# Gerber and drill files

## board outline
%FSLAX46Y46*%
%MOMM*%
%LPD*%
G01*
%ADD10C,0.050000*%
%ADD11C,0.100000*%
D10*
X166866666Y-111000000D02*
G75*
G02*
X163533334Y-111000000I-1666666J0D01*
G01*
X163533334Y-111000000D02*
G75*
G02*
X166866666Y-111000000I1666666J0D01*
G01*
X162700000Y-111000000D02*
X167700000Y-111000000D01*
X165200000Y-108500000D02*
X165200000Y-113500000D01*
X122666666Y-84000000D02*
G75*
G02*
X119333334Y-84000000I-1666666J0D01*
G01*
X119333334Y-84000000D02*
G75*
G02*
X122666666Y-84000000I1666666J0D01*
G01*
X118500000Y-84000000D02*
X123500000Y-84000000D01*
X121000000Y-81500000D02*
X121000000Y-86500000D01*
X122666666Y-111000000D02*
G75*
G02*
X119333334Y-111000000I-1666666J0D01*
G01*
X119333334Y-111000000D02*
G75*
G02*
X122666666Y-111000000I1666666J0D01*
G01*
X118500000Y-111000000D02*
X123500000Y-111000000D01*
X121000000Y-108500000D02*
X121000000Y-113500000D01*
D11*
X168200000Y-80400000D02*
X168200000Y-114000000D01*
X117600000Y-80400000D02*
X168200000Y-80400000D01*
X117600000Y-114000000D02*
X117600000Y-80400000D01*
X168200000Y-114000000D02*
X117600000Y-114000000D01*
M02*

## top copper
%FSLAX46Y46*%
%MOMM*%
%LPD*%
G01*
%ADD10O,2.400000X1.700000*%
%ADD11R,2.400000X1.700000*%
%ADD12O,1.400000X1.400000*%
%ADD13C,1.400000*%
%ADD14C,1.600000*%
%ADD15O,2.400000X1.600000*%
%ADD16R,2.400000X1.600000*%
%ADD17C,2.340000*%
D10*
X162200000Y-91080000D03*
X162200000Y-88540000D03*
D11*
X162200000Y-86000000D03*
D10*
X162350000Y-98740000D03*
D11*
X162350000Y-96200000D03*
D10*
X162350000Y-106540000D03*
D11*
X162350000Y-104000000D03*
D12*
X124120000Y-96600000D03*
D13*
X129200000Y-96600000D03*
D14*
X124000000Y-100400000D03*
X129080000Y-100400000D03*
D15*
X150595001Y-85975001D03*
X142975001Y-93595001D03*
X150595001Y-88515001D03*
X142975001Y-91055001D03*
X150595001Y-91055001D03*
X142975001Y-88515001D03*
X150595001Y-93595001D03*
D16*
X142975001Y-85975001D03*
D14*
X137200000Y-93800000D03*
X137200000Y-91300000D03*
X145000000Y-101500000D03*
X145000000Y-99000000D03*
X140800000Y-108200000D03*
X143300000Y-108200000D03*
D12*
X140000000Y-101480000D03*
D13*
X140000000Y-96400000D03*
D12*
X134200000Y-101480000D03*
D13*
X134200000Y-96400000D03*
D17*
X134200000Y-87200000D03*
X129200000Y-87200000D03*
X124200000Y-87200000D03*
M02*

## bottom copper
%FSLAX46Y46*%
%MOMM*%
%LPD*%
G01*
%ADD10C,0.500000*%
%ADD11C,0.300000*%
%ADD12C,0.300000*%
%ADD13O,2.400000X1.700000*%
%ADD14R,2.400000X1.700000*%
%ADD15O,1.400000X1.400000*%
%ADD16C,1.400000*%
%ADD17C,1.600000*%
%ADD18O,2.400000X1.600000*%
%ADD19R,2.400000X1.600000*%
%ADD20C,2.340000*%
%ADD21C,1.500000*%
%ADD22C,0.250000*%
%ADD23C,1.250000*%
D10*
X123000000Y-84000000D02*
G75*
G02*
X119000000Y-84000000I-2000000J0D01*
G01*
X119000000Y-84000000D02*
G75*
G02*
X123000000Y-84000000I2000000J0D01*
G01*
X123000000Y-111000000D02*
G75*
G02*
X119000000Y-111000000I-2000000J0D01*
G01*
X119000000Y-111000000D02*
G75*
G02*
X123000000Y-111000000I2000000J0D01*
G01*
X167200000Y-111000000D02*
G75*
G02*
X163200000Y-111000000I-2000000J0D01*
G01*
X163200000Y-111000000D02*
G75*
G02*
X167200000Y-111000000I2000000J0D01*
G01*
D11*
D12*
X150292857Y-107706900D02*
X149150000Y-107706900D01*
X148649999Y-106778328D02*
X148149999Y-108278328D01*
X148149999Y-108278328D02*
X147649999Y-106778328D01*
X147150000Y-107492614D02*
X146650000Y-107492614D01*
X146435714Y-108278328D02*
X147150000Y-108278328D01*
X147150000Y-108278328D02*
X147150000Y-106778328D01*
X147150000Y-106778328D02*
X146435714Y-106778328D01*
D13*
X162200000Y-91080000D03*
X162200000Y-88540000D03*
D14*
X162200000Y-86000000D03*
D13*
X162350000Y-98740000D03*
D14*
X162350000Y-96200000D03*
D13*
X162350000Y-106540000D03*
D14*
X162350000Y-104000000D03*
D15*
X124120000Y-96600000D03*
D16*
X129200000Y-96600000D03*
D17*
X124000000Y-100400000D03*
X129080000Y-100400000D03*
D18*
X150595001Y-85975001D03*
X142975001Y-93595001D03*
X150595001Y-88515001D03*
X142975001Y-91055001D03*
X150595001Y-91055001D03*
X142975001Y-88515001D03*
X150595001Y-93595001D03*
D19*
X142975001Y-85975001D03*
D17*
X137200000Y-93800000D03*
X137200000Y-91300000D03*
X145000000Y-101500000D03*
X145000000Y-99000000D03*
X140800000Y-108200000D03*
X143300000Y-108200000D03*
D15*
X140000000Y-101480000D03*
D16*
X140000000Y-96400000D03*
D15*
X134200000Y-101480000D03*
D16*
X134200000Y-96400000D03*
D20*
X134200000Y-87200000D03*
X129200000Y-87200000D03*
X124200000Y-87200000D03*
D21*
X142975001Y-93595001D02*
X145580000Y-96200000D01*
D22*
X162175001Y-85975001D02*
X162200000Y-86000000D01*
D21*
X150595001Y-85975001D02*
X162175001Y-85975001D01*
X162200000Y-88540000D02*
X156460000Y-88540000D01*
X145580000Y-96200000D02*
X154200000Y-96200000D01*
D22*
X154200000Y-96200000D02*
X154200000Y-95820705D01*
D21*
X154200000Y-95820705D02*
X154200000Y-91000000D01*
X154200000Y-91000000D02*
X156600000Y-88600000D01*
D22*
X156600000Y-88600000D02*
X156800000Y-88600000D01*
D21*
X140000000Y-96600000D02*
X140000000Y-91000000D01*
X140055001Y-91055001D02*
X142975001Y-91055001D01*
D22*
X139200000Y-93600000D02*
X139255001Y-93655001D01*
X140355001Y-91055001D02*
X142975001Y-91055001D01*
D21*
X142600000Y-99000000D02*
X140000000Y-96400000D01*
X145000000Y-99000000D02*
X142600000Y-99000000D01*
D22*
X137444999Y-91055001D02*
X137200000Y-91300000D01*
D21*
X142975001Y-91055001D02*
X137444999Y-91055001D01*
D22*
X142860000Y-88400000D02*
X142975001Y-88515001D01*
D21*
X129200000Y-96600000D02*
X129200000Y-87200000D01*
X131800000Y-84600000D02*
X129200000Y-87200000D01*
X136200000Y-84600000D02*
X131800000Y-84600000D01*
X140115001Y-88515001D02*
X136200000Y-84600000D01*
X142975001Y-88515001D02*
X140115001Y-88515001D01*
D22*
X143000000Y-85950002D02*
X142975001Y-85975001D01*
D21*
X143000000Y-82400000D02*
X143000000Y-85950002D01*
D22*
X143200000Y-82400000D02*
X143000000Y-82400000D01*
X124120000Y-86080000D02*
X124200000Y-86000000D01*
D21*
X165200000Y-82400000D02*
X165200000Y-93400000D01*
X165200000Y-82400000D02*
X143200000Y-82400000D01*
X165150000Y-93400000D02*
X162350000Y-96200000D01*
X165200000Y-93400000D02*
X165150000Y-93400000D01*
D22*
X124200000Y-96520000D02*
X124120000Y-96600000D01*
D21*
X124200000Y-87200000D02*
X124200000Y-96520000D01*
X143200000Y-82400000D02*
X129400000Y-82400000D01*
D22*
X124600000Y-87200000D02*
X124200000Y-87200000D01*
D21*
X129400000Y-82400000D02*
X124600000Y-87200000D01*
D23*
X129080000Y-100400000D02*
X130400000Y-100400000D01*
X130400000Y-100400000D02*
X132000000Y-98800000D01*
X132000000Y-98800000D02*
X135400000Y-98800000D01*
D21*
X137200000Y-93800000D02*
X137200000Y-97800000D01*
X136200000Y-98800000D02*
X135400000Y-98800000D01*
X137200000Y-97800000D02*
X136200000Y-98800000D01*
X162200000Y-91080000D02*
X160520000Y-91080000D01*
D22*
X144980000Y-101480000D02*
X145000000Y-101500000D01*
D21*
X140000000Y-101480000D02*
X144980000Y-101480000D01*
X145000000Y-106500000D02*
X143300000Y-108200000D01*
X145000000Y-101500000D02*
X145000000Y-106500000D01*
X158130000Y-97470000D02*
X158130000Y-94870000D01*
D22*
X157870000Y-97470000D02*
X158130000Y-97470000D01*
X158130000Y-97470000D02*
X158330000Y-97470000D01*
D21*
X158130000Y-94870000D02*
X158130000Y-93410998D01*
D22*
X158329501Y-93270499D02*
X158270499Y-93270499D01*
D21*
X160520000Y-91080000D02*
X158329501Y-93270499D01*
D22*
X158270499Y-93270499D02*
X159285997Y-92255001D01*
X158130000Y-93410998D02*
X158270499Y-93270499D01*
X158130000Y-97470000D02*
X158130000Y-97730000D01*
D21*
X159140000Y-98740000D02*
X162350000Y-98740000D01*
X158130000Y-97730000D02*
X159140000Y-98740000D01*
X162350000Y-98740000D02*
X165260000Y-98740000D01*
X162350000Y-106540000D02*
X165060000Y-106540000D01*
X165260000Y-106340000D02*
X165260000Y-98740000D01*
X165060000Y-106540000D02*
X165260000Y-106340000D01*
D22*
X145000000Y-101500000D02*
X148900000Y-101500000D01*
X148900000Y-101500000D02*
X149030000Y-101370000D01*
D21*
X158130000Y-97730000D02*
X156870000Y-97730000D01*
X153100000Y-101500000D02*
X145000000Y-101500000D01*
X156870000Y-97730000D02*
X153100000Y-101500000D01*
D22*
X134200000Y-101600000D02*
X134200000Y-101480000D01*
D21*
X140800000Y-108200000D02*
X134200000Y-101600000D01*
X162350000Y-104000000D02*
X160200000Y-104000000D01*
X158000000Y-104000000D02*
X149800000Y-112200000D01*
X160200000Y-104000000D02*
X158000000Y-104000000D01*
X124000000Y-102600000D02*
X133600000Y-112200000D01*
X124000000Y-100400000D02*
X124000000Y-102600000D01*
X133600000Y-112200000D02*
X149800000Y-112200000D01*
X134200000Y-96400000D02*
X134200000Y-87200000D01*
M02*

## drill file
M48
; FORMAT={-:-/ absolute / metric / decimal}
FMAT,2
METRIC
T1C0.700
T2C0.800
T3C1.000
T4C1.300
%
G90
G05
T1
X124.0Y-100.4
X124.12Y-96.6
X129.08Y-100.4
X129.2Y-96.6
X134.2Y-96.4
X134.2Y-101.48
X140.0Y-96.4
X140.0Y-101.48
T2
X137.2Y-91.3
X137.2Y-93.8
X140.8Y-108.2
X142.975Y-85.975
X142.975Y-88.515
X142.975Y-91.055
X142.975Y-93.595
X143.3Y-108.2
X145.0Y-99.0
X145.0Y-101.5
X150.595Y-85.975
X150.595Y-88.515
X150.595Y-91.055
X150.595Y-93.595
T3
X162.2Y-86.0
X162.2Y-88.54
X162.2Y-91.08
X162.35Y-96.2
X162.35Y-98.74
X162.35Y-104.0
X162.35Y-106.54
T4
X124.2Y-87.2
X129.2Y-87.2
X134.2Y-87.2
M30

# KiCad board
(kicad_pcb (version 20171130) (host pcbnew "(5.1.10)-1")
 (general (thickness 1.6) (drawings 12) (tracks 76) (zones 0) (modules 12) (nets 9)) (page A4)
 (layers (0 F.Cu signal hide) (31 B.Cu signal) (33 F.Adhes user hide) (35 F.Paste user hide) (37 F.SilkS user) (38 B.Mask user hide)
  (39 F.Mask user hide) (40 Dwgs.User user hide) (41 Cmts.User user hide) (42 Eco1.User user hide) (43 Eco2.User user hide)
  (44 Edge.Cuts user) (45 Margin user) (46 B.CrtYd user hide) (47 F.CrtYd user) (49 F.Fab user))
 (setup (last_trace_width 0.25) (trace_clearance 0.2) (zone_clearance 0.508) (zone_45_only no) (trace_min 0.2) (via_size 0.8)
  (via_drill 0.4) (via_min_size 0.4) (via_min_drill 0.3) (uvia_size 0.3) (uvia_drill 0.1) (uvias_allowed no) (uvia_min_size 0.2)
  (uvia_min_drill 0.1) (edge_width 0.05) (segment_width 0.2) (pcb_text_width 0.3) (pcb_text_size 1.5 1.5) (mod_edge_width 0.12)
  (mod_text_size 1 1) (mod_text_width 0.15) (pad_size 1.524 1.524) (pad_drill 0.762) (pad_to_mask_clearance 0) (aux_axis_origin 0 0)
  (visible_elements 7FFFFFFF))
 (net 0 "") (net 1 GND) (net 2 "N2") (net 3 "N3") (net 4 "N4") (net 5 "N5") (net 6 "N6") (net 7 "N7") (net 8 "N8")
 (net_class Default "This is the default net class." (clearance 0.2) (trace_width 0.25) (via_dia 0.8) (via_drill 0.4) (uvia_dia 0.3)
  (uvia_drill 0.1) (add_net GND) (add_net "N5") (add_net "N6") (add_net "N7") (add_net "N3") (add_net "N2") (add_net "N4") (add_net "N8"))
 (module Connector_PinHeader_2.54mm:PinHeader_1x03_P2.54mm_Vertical (layer F.Cu) (at 162.2 86)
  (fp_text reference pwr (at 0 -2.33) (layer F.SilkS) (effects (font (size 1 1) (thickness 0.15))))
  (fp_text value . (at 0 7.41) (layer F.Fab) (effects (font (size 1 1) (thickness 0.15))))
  (pad 3 thru_hole oval (at 0 5.08) (size 2.4 1.7) (drill 1) (layers *.Cu *.Mask) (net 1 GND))
  (pad 2 thru_hole oval (at 0 2.54) (size 2.4 1.7) (drill 1) (layers *.Cu *.Mask))
  (pad 1 thru_hole rect (at 0 0) (size 2.4 1.7) (drill 1) (layers *.Cu *.Mask)))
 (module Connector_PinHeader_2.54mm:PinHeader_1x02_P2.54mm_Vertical (layer F.Cu) (at 162.35 96.2)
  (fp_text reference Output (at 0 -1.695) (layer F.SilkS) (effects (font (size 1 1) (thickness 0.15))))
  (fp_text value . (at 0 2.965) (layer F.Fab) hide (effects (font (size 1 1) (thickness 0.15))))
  (pad 2 thru_hole oval (at 0 2.54) (size 2.4 1.7) (drill 1) (layers *.Cu *.Mask) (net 1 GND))
  (pad 1 thru_hole rect (at 0 0) (size 2.4 1.7) (drill 1) (layers *.Cu *.Mask) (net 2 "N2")))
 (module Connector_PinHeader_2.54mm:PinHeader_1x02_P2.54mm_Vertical (layer F.Cu) (at 162.35 104)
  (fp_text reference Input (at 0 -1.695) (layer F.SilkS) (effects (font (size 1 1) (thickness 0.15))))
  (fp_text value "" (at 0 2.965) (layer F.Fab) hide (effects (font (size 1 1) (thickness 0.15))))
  (pad 2 thru_hole oval (at 0 2.54) (size 2.4 1.7) (drill 1) (layers *.Cu *.Mask) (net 1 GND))
  (pad 1 thru_hole rect (at 0 0) (size 2.4 1.7) (drill 1) (layers *.Cu *.Mask) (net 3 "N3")))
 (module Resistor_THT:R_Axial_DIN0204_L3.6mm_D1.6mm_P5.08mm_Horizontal (layer F.Cu) (at 129.2 96.6 180)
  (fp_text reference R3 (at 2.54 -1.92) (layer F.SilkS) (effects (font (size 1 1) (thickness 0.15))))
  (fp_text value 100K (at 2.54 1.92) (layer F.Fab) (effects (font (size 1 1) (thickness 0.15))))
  (pad 2 thru_hole oval (at 5.08 0 180) (size 1.4 1.4) (drill 0.7) (layers *.Cu *.Mask) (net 2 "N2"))
  (pad 1 thru_hole circle (at 0 0 180) (size 1.4 1.4) (drill 0.7) (layers *.Cu *.Mask) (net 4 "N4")))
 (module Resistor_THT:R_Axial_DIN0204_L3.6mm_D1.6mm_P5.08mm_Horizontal (layer F.Cu) (at 124 100.4)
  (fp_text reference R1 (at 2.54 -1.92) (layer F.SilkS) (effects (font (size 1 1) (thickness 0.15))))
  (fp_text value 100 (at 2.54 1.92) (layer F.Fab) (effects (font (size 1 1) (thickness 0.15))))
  (pad 1 thru_hole circle (at 0 0) (size 1.6 1.6) (drill 0.7) (layers *.Cu *.Mask) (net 3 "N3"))
  (pad 2 thru_hole circle (at 5.08 0) (size 1.6 1.6) (drill 0.7) (layers *.Cu *.Mask) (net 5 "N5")))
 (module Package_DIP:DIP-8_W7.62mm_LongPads (layer F.Cu) (at 142.975001 85.975001)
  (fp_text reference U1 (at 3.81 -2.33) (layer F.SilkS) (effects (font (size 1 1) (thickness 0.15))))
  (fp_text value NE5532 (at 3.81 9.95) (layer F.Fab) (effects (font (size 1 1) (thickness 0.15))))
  (pad 8 thru_hole oval (at 7.62 0) (size 2.4 1.6) (drill 0.8) (layers *.Cu *.Mask))
  (pad 4 thru_hole oval (at 0 7.62) (size 2.4 1.6) (drill 0.8) (layers *.Cu *.Mask))
  (pad 7 thru_hole oval (at 7.62 2.54) (size 2.4 1.6) (drill 0.8) (layers *.Cu *.Mask))
  (pad 3 thru_hole oval (at 0 5.08) (size 2.4 1.6) (drill 0.8) (layers *.Cu *.Mask) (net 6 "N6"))
  (pad 6 thru_hole oval (at 7.62 5.08) (size 2.4 1.6) (drill 0.8) (layers *.Cu *.Mask))
  (pad 2 thru_hole oval (at 0 2.54) (size 2.4 1.6) (drill 0.8) (layers *.Cu *.Mask) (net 4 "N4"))
  (pad 5 thru_hole oval (at 7.62 7.62) (size 2.4 1.6) (drill 0.8) (layers *.Cu *.Mask))
  (pad 1 thru_hole rect (at 0 0) (size 2.4 1.6) (drill 0.8) (layers *.Cu *.Mask) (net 2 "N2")))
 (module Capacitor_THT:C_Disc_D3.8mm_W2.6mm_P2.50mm (layer F.Cu) (at 137.2 93.8 90)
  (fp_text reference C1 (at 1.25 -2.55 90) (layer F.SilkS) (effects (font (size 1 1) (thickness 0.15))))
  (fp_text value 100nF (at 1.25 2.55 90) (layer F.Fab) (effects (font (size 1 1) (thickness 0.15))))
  (pad 1 thru_hole circle (at 0 0 90) (size 1.6 1.6) (drill 0.8) (layers *.Cu *.Mask) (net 5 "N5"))
  (pad 2 thru_hole circle (at 2.5 0 90) (size 1.6 1.6) (drill 0.8) (layers *.Cu *.Mask) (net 6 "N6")))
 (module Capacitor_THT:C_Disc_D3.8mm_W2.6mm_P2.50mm (layer F.Cu) (at 145 99 270)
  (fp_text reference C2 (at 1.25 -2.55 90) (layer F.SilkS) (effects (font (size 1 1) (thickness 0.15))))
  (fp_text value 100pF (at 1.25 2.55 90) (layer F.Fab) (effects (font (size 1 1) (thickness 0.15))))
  (pad 2 thru_hole circle (at 2.5 0 270) (size 1.6 1.6) (drill 0.8) (layers *.Cu *.Mask) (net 1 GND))
  (pad 1 thru_hole circle (at 0 0 270) (size 1.6 1.6) (drill 0.8) (layers *.Cu *.Mask) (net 6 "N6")))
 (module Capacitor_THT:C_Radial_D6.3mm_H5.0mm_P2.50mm (layer F.Cu) (at 140.8 108.2)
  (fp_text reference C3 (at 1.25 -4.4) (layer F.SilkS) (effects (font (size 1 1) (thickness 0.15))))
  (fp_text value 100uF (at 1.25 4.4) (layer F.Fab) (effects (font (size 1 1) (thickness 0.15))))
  (pad 1 thru_hole circle (at 0 0) (size 1.6 1.6) (drill 0.8) (layers *.Cu *.Mask) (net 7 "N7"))
  (pad 2 thru_hole circle (at 2.5 0) (size 1.6 1.6) (drill 0.8) (layers *.Cu *.Mask) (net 1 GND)))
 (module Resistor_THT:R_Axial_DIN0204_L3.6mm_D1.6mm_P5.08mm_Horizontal (layer F.Cu) (at 140 96.4 270)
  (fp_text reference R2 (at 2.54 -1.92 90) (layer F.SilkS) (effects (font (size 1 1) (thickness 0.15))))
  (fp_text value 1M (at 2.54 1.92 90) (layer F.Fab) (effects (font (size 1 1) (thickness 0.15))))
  (pad 2 thru_hole oval (at 5.08 0 270) (size 1.4 1.4) (drill 0.7) (layers *.Cu *.Mask) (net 1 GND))
  (pad 1 thru_hole circle (at 0 0 270) (size 1.4 1.4) (drill 0.7) (layers *.Cu *.Mask) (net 6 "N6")))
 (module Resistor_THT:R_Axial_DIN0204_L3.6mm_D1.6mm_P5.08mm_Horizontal (layer F.Cu) (at 134.2 96.4 270)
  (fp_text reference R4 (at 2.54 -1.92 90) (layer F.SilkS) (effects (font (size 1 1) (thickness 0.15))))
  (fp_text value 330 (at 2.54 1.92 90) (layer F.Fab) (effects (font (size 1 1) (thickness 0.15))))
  (pad 2 thru_hole oval (at 5.08 0 270) (size 1.4 1.4) (drill 0.7) (layers *.Cu *.Mask) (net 7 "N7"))
  (pad 1 thru_hole circle (at 0 0 270) (size 1.4 1.4) (drill 0.7) (layers *.Cu *.Mask) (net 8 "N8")))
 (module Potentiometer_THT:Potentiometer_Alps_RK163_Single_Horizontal (layer B.Cu) (at 124.2 87.2 90)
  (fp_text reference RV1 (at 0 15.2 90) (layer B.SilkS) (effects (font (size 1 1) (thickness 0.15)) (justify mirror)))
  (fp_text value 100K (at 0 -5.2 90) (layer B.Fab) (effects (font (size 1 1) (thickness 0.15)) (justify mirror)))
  (pad 3 thru_hole circle (at 0 10 90) (size 2.34 2.34) (drill 1.3) (layers *.Cu *.Mask) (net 8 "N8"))
  (pad 2 thru_hole circle (at 0 5 90) (size 2.34 2.34) (drill 1.3) (layers *.Cu *.Mask) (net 4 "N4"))
  (pad 1 thru_hole circle (at 0 0 90) (size 2.34 2.34) (drill 1.3) (layers *.Cu *.Mask) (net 2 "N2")))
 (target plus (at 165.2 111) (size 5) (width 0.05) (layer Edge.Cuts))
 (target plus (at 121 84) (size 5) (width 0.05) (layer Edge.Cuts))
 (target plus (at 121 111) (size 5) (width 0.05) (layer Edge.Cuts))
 (gr_circle (center 121 84) (end 123 84) (layer B.Cu) (width 0.5))
 (gr_circle (center 121 111) (end 123 111) (layer B.Cu) (width 0.5))
 (gr_circle (center 165.2 111) (end 167.2 111) (layer B.Cu) (width 0.5))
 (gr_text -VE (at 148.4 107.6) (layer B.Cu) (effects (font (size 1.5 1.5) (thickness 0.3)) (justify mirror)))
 (gr_line (start 168.2 80.4) (end 168.2 114) (layer Edge.Cuts) (width 0.1))
 (gr_line (start 117.6 80.4) (end 168.2 80.4) (layer Edge.Cuts) (width 0.1))
 (gr_line (start 117.6 114) (end 117.6 80.4) (layer Edge.Cuts) (width 0.1))
 (gr_line (start 168.2 114) (end 117.6 114) (layer Edge.Cuts) (width 0.1))
 (segment (start 142.975001 93.595001) (end 145.58 96.2) (width 1.5) (layer B.Cu) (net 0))
 (segment (start 162.175001 85.975001) (end 162.2 86) (width 0.25) (layer B.Cu) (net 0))
 (segment (start 150.595001 85.975001) (end 162.175001 85.975001) (width 1.5) (layer B.Cu) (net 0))
 (segment (start 162.2 88.54) (end 156.46 88.54) (width 1.5) (layer B.Cu) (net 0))
 (segment (start 145.58 96.2) (end 154.2 96.2) (width 1.5) (layer B.Cu) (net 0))
 (segment (start 154.2 96.2) (end 154.2 95.820705) (width 0.25) (layer B.Cu) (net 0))
 (segment (start 154.2 95.820705) (end 154.2 91) (width 1.5) (layer B.Cu) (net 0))
 (segment (start 154.2 91) (end 156.6 88.6) (width 1.5) (layer B.Cu) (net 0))
 (segment (start 156.6 88.6) (end 156.8 88.6) (width 0.25) (layer B.Cu) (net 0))
 (segment (start 140 96.6) (end 140 91) (width 1.5) (layer B.Cu) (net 6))
 (segment (start 140.055001 91.055001) (end 142.975001 91.055001) (width 1.5) (layer B.Cu) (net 6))
 (segment (start 139.2 93.6) (end 139.255001 93.655001) (width 0.25) (layer B.Cu) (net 6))
 (segment (start 140.355001 91.055001) (end 142.975001 91.055001) (width 0.25) (layer B.Cu) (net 6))
 (segment (start 142.6 99) (end 140 96.4) (width 1.5) (layer B.Cu) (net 6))
 (segment (start 145 99) (end 142.6 99) (width 1.5) (layer B.Cu) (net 6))
 (segment (start 137.444999 91.055001) (end 137.2 91.3) (width 0.25) (layer B.Cu) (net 6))
 (segment (start 142.975001 91.055001) (end 137.444999 91.055001) (width 1.5) (layer B.Cu) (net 6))
 (segment (start 142.86 88.4) (end 142.975001 88.515001) (width 0.25) (layer B.Cu) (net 4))
 (segment (start 129.2 96.6) (end 129.2 87.2) (width 1.5) (layer B.Cu) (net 4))
 (segment (start 131.8 84.6) (end 129.2 87.2) (width 1.5) (layer B.Cu) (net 4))
 (segment (start 136.2 84.6) (end 131.8 84.6) (width 1.5) (layer B.Cu) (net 4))
 (segment (start 140.115001 88.515001) (end 136.2 84.6) (width 1.5) (layer B.Cu) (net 4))
 (segment (start 142.975001 88.515001) (end 140.115001 88.515001) (width 1.5) (layer B.Cu) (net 4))
 (segment (start 143 85.950002) (end 142.975001 85.975001) (width 0.25) (layer B.Cu) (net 2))
 (segment (start 143 82.4) (end 143 85.950002) (width 1.5) (layer B.Cu) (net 2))
 (segment (start 143.2 82.4) (end 143 82.4) (width 0.25) (layer B.Cu) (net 2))
 (segment (start 124.12 86.08) (end 124.2 86) (width 0.25) (layer B.Cu) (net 2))
 (segment (start 165.2 82.4) (end 165.2 93.4) (width 1.5) (layer B.Cu) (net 2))
 (segment (start 165.2 82.4) (end 143.2 82.4) (width 1.5) (layer B.Cu) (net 2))
 (segment (start 165.15 93.4) (end 162.35 96.2) (width 1.5) (layer B.Cu) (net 2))
 (segment (start 165.2 93.4) (end 165.15 93.4) (width 1.5) (layer B.Cu) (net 2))
 (segment (start 124.2 96.52) (end 124.12 96.6) (width 0.25) (layer B.Cu) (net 2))
 (segment (start 124.2 87.2) (end 124.2 96.52) (width 1.5) (layer B.Cu) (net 2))
 (segment (start 143.2 82.4) (end 129.4 82.4) (width 1.5) (layer B.Cu) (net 2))
 (segment (start 124.6 87.2) (end 124.2 87.2) (width 0.25) (layer B.Cu) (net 2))
 (segment (start 129.4 82.4) (end 124.6 87.2) (width 1.5) (layer B.Cu) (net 2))
 (segment (start 129.08 100.4) (end 130.4 100.4) (width 1.25) (layer B.Cu) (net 5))
 (segment (start 130.4 100.4) (end 132 98.8) (width 1.25) (layer B.Cu) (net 5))
 (segment (start 132 98.8) (end 135.4 98.8) (width 1.25) (layer B.Cu) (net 5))
 (segment (start 137.2 93.8) (end 137.2 97.8) (width 1.5) (layer B.Cu) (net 5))
 (segment (start 136.2 98.8) (end 135.4 98.8) (width 1.5) (layer B.Cu) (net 5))
 (segment (start 137.2 97.8) (end 136.2 98.8) (width 1.5) (layer B.Cu) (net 5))
 (segment (start 162.2 91.08) (end 160.52 91.08) (width 1.5) (layer B.Cu) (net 1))
 (segment (start 144.98 101.48) (end 145 101.5) (width 0.25) (layer B.Cu) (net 1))
 (segment (start 140 101.48) (end 144.98 101.48) (width 1.5) (layer B.Cu) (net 1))
 (segment (start 145 106.5) (end 143.3 108.2) (width 1.5) (layer B.Cu) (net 1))
 (segment (start 145 101.5) (end 145 106.5) (width 1.5) (layer B.Cu) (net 1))
 (segment (start 158.13 97.47) (end 158.13 94.87) (width 1.5) (layer B.Cu) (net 1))
 (segment (start 157.87 97.47) (end 158.13 97.47) (width 0.25) (layer B.Cu) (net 1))
 (segment (start 158.13 97.47) (end 158.33 97.47) (width 0.25) (layer B.Cu) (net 1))
 (segment (start 158.13 94.87) (end 158.13 93.410998) (width 1.5) (layer B.Cu) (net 1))
 (segment (start 158.329501 93.270499) (end 158.270499 93.270499) (width 0.25) (layer B.Cu) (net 1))
 (segment (start 160.52 91.08) (end 158.329501 93.270499) (width 1.5) (layer B.Cu) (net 1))
 (segment (start 158.270499 93.270499) (end 159.285997 92.255001) (width 0.25) (layer B.Cu) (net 1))
 (segment (start 158.13 93.410998) (end 158.270499 93.270499) (width 0.25) (layer B.Cu) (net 1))
 (segment (start 158.13 97.47) (end 158.13 97.73) (width 0.25) (layer B.Cu) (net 1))
 (segment (start 159.14 98.74) (end 162.35 98.74) (width 1.5) (layer B.Cu) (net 1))
 (segment (start 158.13 97.73) (end 159.14 98.74) (width 1.5) (layer B.Cu) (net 1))
 (segment (start 162.35 98.74) (end 165.26 98.74) (width 1.5) (layer B.Cu) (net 1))
 (segment (start 162.35 106.54) (end 165.06 106.54) (width 1.5) (layer B.Cu) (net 1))
 (segment (start 165.26 106.34) (end 165.26 98.74) (width 1.5) (layer B.Cu) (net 1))
 (segment (start 165.06 106.54) (end 165.26 106.34) (width 1.5) (layer B.Cu) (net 1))
 (segment (start 145 101.5) (end 148.9 101.5) (width 0.25) (layer B.Cu) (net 1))
 (segment (start 148.9 101.5) (end 149.03 101.37) (width 0.25) (layer B.Cu) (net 1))
 (segment (start 158.13 97.73) (end 156.87 97.73) (width 1.5) (layer B.Cu) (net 1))
 (segment (start 153.1 101.5) (end 145 101.5) (width 1.5) (layer B.Cu) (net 1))
 (segment (start 156.87 97.73) (end 153.1 101.5) (width 1.5) (layer B.Cu) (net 1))
 (segment (start 134.2 101.6) (end 134.2 101.48) (width 0.25) (layer B.Cu) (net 7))
 (segment (start 140.8 108.2) (end 134.2 101.6) (width 1.5) (layer B.Cu) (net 7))
 (segment (start 162.35 104) (end 160.2 104) (width 1.5) (layer B.Cu) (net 3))
 (segment (start 158 104) (end 149.8 112.2) (width 1.5) (layer B.Cu) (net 3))
 (segment (start 160.2 104) (end 158 104) (width 1.5) (layer B.Cu) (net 3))
 (segment (start 124 102.6) (end 133.6 112.2) (width 1.5) (layer B.Cu) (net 3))
 (segment (start 124 100.4) (end 124 102.6) (width 1.5) (layer B.Cu) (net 3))
 (segment (start 133.6 112.2) (end 149.8 112.2) (width 1.5) (layer B.Cu) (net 3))
 (segment (start 134.2 96.4) (end 134.2 87.2) (width 1.5) (layer B.Cu) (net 8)))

